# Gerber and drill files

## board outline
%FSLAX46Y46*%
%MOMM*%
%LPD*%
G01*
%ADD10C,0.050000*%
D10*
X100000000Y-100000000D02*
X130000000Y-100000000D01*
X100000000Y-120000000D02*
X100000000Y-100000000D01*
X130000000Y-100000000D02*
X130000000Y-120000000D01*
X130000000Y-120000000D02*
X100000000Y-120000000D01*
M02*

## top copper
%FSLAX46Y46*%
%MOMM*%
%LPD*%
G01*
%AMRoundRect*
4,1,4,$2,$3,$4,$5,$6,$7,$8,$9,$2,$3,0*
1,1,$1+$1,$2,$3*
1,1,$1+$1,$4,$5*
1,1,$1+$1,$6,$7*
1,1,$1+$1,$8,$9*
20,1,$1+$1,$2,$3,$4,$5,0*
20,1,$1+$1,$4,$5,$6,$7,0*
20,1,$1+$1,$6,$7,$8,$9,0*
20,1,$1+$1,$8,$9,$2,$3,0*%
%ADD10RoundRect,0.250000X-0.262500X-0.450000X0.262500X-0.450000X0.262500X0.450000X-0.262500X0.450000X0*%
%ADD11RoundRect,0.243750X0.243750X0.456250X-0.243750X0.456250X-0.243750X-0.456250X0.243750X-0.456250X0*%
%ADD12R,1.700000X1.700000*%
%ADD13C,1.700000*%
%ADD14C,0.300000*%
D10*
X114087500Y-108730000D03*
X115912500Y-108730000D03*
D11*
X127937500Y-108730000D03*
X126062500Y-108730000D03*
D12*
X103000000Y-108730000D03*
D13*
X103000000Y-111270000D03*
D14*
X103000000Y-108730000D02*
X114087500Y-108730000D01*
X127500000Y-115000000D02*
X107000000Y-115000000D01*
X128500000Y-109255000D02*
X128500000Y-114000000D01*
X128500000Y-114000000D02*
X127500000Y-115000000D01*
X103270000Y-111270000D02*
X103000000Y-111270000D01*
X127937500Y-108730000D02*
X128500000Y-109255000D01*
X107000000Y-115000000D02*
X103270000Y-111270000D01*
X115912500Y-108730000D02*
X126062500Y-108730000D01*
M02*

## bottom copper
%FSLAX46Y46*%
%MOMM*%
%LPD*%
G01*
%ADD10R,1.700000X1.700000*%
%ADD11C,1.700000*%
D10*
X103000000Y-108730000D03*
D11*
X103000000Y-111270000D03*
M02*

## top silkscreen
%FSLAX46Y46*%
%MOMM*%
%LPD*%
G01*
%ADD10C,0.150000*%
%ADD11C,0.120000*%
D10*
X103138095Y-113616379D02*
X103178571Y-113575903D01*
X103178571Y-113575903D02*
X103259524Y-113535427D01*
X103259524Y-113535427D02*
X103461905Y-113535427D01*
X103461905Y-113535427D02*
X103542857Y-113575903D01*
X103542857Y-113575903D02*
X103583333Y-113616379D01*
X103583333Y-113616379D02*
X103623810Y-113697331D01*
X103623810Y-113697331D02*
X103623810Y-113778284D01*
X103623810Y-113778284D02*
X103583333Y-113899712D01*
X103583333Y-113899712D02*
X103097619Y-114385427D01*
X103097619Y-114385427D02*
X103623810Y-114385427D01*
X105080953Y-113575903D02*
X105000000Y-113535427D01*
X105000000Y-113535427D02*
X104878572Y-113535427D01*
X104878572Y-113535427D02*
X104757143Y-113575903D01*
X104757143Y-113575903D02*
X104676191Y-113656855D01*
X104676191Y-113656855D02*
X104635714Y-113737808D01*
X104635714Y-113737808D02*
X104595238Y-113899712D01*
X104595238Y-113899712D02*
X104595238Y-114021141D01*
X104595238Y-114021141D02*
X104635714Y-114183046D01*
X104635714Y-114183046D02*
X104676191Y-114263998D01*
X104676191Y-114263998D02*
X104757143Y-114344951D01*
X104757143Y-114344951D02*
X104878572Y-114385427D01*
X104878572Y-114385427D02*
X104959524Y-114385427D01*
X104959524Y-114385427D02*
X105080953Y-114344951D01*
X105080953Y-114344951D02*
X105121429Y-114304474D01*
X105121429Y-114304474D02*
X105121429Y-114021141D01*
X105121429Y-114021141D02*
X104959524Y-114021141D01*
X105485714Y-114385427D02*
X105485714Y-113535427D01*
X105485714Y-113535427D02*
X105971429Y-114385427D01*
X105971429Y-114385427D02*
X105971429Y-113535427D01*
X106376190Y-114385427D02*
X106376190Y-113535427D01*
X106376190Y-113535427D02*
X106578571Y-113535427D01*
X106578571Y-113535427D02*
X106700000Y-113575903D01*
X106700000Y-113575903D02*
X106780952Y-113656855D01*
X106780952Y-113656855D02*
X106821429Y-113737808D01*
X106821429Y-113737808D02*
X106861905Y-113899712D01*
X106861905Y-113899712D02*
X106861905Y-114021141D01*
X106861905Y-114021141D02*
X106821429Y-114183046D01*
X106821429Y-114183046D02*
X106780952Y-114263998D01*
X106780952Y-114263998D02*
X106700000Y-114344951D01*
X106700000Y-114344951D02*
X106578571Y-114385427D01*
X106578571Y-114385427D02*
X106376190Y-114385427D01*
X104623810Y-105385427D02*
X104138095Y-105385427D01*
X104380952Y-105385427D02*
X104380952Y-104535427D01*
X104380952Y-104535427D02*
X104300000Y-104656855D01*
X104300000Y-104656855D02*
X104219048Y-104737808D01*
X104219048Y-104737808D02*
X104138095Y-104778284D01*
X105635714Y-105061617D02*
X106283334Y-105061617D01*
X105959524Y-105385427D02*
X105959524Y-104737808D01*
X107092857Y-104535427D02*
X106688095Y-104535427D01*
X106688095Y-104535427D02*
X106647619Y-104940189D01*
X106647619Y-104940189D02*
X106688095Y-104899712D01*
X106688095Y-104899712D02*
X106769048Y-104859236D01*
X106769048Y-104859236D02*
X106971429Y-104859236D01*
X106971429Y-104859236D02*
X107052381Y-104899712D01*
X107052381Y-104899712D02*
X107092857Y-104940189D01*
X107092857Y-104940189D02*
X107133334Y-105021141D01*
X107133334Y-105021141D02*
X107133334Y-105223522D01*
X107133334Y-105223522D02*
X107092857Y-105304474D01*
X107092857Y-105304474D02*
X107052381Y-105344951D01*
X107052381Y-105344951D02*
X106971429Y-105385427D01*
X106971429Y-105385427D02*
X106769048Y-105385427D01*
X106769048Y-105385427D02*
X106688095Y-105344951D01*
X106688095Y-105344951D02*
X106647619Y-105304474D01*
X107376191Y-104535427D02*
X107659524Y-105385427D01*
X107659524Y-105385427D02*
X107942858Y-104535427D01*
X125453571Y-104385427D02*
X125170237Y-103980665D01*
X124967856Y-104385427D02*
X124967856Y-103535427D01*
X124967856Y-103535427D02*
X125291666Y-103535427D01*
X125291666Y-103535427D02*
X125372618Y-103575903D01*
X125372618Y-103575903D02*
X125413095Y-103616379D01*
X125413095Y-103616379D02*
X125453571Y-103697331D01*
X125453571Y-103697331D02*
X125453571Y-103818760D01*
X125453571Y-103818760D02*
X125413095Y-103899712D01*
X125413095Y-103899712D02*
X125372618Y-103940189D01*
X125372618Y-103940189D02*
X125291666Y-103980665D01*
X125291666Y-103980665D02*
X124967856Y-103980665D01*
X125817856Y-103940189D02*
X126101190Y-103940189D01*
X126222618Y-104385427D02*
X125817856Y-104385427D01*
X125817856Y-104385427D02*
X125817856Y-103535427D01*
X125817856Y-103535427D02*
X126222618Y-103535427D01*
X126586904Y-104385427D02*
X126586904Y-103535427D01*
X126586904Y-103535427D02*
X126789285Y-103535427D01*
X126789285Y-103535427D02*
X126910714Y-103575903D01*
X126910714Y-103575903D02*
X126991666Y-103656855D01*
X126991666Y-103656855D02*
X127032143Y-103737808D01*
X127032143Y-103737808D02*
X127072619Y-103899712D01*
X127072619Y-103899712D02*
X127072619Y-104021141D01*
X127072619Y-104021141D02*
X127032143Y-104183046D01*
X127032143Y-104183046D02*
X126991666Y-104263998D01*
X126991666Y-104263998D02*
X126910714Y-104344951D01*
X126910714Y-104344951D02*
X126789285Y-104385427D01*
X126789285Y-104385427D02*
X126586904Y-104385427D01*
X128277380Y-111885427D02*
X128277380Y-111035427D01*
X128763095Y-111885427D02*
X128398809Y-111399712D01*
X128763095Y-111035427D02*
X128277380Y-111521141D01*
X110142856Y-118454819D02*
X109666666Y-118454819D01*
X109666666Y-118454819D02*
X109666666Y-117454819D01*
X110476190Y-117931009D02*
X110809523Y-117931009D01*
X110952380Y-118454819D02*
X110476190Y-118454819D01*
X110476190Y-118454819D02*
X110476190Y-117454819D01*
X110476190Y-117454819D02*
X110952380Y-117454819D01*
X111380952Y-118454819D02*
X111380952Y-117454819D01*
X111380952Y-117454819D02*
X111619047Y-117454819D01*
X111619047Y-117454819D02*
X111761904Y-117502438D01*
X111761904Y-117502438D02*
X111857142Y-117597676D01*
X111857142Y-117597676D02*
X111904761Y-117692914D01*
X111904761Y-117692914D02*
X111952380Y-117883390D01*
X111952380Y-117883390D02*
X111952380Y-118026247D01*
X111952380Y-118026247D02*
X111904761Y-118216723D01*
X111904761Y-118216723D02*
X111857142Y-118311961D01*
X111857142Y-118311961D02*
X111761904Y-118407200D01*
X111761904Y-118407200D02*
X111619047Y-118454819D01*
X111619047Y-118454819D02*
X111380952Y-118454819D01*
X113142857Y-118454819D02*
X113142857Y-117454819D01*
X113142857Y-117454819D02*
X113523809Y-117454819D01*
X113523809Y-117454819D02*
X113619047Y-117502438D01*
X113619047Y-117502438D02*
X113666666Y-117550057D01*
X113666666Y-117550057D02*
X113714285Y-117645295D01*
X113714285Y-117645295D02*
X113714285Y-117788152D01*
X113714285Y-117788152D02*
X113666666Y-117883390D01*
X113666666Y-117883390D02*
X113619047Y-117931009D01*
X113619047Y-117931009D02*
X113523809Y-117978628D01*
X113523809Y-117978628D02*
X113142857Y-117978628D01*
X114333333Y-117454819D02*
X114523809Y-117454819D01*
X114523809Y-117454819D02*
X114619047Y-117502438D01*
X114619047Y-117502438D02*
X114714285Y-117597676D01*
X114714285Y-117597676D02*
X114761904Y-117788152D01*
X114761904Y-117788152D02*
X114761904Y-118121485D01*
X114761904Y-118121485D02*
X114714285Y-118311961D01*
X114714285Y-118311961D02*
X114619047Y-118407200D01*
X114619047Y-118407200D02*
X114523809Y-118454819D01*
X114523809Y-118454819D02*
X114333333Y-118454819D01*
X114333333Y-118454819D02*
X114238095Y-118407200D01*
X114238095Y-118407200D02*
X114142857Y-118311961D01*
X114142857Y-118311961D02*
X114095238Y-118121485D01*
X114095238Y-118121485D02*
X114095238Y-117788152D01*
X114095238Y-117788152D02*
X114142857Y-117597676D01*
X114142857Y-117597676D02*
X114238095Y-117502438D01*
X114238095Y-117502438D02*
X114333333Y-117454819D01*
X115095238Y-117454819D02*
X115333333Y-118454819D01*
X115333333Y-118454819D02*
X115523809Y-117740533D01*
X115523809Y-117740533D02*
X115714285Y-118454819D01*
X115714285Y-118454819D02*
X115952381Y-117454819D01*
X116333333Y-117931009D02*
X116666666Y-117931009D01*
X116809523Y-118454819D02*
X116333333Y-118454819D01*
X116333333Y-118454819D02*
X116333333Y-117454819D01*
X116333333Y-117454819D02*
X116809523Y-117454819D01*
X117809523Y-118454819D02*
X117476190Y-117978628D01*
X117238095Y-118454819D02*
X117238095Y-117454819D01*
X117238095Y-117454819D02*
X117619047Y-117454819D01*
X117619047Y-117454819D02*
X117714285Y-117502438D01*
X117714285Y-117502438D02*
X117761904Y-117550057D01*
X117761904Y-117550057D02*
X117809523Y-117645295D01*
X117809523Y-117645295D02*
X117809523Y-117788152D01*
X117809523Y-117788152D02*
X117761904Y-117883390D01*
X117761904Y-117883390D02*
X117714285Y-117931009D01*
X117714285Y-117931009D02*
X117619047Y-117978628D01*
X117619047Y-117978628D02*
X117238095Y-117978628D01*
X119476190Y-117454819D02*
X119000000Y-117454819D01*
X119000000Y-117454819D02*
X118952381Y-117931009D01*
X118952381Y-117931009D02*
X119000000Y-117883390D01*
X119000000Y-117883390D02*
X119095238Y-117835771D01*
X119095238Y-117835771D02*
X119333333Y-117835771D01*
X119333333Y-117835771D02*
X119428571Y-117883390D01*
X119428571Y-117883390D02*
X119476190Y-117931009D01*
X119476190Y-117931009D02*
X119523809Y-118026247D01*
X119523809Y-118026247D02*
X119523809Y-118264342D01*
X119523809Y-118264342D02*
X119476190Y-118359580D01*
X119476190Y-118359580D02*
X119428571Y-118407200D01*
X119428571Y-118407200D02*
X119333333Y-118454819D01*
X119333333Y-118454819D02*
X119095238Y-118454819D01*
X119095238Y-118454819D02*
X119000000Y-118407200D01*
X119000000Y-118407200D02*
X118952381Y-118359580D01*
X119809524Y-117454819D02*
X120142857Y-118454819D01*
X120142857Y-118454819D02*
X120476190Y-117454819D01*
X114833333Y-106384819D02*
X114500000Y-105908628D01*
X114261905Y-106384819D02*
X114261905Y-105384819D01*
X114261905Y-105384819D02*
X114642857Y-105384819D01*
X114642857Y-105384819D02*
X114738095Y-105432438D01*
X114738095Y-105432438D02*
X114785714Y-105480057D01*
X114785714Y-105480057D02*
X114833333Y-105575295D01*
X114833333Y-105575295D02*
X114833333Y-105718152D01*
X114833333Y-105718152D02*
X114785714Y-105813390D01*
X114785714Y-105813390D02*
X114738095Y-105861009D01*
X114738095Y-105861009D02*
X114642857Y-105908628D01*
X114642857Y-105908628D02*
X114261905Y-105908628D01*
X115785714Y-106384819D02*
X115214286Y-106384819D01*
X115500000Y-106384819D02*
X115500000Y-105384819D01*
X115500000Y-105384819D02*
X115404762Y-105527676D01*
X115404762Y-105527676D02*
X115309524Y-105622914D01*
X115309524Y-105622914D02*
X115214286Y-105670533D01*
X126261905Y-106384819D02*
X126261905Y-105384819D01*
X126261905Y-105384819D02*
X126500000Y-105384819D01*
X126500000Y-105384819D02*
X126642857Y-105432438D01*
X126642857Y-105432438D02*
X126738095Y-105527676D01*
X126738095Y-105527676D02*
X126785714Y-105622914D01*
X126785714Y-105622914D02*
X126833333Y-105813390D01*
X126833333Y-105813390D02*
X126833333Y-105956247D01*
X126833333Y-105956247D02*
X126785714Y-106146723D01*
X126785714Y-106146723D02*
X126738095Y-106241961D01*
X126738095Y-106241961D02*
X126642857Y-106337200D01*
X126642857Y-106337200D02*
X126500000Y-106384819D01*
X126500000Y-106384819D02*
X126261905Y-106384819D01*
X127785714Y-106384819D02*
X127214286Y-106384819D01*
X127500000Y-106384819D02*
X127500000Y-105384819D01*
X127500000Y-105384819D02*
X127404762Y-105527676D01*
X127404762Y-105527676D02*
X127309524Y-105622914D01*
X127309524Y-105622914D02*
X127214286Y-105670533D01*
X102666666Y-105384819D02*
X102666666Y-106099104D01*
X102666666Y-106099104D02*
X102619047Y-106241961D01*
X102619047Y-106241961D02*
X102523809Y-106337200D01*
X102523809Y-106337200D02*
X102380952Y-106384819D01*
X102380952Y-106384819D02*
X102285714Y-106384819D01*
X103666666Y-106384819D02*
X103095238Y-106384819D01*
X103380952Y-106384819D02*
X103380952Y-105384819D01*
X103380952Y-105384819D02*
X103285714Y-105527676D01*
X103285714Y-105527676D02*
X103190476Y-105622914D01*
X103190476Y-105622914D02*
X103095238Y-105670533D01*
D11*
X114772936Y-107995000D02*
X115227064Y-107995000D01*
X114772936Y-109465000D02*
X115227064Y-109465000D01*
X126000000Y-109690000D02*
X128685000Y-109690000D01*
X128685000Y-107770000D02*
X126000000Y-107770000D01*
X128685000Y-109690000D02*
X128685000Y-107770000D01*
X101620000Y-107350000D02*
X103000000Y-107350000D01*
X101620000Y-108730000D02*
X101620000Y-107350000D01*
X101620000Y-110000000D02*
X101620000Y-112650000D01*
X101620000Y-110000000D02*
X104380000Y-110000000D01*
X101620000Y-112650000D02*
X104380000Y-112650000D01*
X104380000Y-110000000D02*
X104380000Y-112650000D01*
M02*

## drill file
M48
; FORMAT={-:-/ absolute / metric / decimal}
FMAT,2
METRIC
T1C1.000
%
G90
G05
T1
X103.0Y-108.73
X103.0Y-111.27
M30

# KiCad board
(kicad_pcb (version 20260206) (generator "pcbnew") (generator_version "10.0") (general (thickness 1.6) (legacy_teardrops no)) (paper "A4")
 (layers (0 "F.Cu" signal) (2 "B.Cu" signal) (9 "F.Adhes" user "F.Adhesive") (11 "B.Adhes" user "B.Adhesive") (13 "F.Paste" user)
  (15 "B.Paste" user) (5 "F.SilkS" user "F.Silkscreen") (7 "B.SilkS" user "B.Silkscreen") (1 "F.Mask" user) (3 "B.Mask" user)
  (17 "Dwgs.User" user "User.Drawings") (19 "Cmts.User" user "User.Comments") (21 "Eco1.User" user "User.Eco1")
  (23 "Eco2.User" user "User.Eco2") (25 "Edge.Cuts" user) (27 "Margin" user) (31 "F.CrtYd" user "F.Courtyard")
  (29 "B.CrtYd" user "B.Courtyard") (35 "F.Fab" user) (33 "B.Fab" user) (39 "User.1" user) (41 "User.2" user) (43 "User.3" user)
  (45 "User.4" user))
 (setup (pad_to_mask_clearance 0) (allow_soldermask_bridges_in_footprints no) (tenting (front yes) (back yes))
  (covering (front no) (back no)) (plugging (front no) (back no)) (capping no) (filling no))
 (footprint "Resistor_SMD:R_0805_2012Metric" (layer "F.Cu") (at 115 108.73)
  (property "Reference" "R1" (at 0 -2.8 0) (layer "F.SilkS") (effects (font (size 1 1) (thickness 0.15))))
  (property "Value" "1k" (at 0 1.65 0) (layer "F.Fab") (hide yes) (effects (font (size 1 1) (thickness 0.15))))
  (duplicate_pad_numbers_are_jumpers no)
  (fp_line (start -0.227064 -0.735) (end 0.227064 -0.735) (stroke (width 0.12) (type solid)) (layer "F.SilkS"))
  (fp_line (start -0.227064 0.735) (end 0.227064 0.735) (stroke (width 0.12) (type solid)) (layer "F.SilkS"))
  (pad "1" smd roundrect (at -0.9125 0) (size 1.025 1.4) (layers "F.Cu" "F.Mask" "F.Paste") (roundrect_rratio 0.243902) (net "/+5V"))
  (pad "2" smd roundrect (at 0.9125 0) (size 1.025 1.4) (layers "F.Cu" "F.Mask" "F.Paste") (roundrect_rratio 0.243902) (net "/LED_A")))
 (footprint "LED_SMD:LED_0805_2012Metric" (layer "F.Cu") (at 127 108.73 180)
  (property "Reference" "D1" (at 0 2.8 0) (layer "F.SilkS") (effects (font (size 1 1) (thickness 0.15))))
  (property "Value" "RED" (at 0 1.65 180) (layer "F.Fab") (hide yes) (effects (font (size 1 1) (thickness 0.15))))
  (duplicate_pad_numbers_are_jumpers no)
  (fp_line (start 1 -0.96) (end -1.685 -0.96) (stroke (width 0.12) (type solid)) (layer "F.SilkS"))
  (fp_line (start -1.685 0.96) (end 1 0.96) (stroke (width 0.12) (type solid)) (layer "F.SilkS"))
  (fp_line (start -1.685 -0.96) (end -1.685 0.96) (stroke (width 0.12) (type solid)) (layer "F.SilkS"))
  (pad "1" smd roundrect (at -0.9375 0 180) (size 0.975 1.4) (layers "F.Cu" "F.Mask" "F.Paste") (roundrect_rratio 0.25) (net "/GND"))
  (pad "2" smd roundrect (at 0.9375 0 180) (size 0.975 1.4) (layers "F.Cu" "F.Mask" "F.Paste") (roundrect_rratio 0.25) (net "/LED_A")))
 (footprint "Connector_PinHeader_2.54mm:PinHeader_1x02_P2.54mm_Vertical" (layer "F.Cu") (at 103 108.73)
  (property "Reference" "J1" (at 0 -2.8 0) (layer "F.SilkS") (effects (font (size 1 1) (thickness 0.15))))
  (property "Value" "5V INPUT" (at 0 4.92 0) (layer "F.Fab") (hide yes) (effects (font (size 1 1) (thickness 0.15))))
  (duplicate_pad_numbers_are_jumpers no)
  (fp_line (start -1.38 -1.38) (end 0 -1.38) (stroke (width 0.12) (type solid)) (layer "F.SilkS"))
  (fp_line (start -1.38 0) (end -1.38 -1.38) (stroke (width 0.12) (type solid)) (layer "F.SilkS"))
  (fp_line (start -1.38 1.27) (end -1.38 3.92) (stroke (width 0.12) (type solid)) (layer "F.SilkS"))
  (fp_line (start -1.38 1.27) (end 1.38 1.27) (stroke (width 0.12) (type solid)) (layer "F.SilkS"))
  (fp_line (start -1.38 3.92) (end 1.38 3.92) (stroke (width 0.12) (type solid)) (layer "F.SilkS"))
  (fp_line (start 1.38 1.27) (end 1.38 3.92) (stroke (width 0.12) (type solid)) (layer "F.SilkS"))
  (pad "1" thru_hole rect (at 0 0) (size 1.7 1.7) (drill 1) (layers "*.Cu" "*.Mask") (remove_unused_layers no) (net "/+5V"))
  (pad "2" thru_hole circle (at 0 2.54) (size 1.7 1.7) (drill 1) (layers "*.Cu" "*.Mask") (remove_unused_layers no) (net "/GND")))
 (gr_line (start 100 100) (end 130 100) (stroke (width 0.05) (type default)) (layer "Edge.Cuts"))
 (gr_line (start 100 120) (end 100 100) (stroke (width 0.05) (type default)) (layer "Edge.Cuts"))
 (gr_line (start 130 100) (end 130 120) (stroke (width 0.05) (type default)) (layer "Edge.Cuts"))
 (gr_line (start 130 120) (end 100 120) (stroke (width 0.05) (type default)) (layer "Edge.Cuts"))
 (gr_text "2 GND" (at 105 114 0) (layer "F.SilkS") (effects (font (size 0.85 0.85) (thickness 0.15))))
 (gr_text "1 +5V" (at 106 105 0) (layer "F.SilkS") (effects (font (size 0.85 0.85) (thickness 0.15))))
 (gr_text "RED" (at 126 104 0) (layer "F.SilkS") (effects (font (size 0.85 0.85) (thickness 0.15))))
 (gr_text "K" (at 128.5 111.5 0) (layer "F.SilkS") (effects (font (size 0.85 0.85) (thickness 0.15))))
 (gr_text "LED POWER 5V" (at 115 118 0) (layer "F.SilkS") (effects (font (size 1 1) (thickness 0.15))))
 (segment (start 103 108.73) (end 114.0875 108.73) (width 0.3) (layer "F.Cu") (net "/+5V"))
 (segment (start 127.5 115) (end 107 115) (width 0.3) (layer "F.Cu") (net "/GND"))
 (segment (start 128.5 109.255) (end 128.5 114) (width 0.3) (layer "F.Cu") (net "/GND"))
 (segment (start 128.5 114) (end 127.5 115) (width 0.3) (layer "F.Cu") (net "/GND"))
 (segment (start 103.27 111.27) (end 103 111.27) (width 0.3) (layer "F.Cu") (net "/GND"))
 (segment (start 127.9375 108.73) (end 128.5 109.255) (width 0.3) (layer "F.Cu") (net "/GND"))
 (segment (start 107 115) (end 103.27 111.27) (width 0.3) (layer "F.Cu") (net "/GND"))
 (segment (start 115.9125 108.73) (end 126.0625 108.73) (width 0.3) (layer "F.Cu") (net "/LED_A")))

